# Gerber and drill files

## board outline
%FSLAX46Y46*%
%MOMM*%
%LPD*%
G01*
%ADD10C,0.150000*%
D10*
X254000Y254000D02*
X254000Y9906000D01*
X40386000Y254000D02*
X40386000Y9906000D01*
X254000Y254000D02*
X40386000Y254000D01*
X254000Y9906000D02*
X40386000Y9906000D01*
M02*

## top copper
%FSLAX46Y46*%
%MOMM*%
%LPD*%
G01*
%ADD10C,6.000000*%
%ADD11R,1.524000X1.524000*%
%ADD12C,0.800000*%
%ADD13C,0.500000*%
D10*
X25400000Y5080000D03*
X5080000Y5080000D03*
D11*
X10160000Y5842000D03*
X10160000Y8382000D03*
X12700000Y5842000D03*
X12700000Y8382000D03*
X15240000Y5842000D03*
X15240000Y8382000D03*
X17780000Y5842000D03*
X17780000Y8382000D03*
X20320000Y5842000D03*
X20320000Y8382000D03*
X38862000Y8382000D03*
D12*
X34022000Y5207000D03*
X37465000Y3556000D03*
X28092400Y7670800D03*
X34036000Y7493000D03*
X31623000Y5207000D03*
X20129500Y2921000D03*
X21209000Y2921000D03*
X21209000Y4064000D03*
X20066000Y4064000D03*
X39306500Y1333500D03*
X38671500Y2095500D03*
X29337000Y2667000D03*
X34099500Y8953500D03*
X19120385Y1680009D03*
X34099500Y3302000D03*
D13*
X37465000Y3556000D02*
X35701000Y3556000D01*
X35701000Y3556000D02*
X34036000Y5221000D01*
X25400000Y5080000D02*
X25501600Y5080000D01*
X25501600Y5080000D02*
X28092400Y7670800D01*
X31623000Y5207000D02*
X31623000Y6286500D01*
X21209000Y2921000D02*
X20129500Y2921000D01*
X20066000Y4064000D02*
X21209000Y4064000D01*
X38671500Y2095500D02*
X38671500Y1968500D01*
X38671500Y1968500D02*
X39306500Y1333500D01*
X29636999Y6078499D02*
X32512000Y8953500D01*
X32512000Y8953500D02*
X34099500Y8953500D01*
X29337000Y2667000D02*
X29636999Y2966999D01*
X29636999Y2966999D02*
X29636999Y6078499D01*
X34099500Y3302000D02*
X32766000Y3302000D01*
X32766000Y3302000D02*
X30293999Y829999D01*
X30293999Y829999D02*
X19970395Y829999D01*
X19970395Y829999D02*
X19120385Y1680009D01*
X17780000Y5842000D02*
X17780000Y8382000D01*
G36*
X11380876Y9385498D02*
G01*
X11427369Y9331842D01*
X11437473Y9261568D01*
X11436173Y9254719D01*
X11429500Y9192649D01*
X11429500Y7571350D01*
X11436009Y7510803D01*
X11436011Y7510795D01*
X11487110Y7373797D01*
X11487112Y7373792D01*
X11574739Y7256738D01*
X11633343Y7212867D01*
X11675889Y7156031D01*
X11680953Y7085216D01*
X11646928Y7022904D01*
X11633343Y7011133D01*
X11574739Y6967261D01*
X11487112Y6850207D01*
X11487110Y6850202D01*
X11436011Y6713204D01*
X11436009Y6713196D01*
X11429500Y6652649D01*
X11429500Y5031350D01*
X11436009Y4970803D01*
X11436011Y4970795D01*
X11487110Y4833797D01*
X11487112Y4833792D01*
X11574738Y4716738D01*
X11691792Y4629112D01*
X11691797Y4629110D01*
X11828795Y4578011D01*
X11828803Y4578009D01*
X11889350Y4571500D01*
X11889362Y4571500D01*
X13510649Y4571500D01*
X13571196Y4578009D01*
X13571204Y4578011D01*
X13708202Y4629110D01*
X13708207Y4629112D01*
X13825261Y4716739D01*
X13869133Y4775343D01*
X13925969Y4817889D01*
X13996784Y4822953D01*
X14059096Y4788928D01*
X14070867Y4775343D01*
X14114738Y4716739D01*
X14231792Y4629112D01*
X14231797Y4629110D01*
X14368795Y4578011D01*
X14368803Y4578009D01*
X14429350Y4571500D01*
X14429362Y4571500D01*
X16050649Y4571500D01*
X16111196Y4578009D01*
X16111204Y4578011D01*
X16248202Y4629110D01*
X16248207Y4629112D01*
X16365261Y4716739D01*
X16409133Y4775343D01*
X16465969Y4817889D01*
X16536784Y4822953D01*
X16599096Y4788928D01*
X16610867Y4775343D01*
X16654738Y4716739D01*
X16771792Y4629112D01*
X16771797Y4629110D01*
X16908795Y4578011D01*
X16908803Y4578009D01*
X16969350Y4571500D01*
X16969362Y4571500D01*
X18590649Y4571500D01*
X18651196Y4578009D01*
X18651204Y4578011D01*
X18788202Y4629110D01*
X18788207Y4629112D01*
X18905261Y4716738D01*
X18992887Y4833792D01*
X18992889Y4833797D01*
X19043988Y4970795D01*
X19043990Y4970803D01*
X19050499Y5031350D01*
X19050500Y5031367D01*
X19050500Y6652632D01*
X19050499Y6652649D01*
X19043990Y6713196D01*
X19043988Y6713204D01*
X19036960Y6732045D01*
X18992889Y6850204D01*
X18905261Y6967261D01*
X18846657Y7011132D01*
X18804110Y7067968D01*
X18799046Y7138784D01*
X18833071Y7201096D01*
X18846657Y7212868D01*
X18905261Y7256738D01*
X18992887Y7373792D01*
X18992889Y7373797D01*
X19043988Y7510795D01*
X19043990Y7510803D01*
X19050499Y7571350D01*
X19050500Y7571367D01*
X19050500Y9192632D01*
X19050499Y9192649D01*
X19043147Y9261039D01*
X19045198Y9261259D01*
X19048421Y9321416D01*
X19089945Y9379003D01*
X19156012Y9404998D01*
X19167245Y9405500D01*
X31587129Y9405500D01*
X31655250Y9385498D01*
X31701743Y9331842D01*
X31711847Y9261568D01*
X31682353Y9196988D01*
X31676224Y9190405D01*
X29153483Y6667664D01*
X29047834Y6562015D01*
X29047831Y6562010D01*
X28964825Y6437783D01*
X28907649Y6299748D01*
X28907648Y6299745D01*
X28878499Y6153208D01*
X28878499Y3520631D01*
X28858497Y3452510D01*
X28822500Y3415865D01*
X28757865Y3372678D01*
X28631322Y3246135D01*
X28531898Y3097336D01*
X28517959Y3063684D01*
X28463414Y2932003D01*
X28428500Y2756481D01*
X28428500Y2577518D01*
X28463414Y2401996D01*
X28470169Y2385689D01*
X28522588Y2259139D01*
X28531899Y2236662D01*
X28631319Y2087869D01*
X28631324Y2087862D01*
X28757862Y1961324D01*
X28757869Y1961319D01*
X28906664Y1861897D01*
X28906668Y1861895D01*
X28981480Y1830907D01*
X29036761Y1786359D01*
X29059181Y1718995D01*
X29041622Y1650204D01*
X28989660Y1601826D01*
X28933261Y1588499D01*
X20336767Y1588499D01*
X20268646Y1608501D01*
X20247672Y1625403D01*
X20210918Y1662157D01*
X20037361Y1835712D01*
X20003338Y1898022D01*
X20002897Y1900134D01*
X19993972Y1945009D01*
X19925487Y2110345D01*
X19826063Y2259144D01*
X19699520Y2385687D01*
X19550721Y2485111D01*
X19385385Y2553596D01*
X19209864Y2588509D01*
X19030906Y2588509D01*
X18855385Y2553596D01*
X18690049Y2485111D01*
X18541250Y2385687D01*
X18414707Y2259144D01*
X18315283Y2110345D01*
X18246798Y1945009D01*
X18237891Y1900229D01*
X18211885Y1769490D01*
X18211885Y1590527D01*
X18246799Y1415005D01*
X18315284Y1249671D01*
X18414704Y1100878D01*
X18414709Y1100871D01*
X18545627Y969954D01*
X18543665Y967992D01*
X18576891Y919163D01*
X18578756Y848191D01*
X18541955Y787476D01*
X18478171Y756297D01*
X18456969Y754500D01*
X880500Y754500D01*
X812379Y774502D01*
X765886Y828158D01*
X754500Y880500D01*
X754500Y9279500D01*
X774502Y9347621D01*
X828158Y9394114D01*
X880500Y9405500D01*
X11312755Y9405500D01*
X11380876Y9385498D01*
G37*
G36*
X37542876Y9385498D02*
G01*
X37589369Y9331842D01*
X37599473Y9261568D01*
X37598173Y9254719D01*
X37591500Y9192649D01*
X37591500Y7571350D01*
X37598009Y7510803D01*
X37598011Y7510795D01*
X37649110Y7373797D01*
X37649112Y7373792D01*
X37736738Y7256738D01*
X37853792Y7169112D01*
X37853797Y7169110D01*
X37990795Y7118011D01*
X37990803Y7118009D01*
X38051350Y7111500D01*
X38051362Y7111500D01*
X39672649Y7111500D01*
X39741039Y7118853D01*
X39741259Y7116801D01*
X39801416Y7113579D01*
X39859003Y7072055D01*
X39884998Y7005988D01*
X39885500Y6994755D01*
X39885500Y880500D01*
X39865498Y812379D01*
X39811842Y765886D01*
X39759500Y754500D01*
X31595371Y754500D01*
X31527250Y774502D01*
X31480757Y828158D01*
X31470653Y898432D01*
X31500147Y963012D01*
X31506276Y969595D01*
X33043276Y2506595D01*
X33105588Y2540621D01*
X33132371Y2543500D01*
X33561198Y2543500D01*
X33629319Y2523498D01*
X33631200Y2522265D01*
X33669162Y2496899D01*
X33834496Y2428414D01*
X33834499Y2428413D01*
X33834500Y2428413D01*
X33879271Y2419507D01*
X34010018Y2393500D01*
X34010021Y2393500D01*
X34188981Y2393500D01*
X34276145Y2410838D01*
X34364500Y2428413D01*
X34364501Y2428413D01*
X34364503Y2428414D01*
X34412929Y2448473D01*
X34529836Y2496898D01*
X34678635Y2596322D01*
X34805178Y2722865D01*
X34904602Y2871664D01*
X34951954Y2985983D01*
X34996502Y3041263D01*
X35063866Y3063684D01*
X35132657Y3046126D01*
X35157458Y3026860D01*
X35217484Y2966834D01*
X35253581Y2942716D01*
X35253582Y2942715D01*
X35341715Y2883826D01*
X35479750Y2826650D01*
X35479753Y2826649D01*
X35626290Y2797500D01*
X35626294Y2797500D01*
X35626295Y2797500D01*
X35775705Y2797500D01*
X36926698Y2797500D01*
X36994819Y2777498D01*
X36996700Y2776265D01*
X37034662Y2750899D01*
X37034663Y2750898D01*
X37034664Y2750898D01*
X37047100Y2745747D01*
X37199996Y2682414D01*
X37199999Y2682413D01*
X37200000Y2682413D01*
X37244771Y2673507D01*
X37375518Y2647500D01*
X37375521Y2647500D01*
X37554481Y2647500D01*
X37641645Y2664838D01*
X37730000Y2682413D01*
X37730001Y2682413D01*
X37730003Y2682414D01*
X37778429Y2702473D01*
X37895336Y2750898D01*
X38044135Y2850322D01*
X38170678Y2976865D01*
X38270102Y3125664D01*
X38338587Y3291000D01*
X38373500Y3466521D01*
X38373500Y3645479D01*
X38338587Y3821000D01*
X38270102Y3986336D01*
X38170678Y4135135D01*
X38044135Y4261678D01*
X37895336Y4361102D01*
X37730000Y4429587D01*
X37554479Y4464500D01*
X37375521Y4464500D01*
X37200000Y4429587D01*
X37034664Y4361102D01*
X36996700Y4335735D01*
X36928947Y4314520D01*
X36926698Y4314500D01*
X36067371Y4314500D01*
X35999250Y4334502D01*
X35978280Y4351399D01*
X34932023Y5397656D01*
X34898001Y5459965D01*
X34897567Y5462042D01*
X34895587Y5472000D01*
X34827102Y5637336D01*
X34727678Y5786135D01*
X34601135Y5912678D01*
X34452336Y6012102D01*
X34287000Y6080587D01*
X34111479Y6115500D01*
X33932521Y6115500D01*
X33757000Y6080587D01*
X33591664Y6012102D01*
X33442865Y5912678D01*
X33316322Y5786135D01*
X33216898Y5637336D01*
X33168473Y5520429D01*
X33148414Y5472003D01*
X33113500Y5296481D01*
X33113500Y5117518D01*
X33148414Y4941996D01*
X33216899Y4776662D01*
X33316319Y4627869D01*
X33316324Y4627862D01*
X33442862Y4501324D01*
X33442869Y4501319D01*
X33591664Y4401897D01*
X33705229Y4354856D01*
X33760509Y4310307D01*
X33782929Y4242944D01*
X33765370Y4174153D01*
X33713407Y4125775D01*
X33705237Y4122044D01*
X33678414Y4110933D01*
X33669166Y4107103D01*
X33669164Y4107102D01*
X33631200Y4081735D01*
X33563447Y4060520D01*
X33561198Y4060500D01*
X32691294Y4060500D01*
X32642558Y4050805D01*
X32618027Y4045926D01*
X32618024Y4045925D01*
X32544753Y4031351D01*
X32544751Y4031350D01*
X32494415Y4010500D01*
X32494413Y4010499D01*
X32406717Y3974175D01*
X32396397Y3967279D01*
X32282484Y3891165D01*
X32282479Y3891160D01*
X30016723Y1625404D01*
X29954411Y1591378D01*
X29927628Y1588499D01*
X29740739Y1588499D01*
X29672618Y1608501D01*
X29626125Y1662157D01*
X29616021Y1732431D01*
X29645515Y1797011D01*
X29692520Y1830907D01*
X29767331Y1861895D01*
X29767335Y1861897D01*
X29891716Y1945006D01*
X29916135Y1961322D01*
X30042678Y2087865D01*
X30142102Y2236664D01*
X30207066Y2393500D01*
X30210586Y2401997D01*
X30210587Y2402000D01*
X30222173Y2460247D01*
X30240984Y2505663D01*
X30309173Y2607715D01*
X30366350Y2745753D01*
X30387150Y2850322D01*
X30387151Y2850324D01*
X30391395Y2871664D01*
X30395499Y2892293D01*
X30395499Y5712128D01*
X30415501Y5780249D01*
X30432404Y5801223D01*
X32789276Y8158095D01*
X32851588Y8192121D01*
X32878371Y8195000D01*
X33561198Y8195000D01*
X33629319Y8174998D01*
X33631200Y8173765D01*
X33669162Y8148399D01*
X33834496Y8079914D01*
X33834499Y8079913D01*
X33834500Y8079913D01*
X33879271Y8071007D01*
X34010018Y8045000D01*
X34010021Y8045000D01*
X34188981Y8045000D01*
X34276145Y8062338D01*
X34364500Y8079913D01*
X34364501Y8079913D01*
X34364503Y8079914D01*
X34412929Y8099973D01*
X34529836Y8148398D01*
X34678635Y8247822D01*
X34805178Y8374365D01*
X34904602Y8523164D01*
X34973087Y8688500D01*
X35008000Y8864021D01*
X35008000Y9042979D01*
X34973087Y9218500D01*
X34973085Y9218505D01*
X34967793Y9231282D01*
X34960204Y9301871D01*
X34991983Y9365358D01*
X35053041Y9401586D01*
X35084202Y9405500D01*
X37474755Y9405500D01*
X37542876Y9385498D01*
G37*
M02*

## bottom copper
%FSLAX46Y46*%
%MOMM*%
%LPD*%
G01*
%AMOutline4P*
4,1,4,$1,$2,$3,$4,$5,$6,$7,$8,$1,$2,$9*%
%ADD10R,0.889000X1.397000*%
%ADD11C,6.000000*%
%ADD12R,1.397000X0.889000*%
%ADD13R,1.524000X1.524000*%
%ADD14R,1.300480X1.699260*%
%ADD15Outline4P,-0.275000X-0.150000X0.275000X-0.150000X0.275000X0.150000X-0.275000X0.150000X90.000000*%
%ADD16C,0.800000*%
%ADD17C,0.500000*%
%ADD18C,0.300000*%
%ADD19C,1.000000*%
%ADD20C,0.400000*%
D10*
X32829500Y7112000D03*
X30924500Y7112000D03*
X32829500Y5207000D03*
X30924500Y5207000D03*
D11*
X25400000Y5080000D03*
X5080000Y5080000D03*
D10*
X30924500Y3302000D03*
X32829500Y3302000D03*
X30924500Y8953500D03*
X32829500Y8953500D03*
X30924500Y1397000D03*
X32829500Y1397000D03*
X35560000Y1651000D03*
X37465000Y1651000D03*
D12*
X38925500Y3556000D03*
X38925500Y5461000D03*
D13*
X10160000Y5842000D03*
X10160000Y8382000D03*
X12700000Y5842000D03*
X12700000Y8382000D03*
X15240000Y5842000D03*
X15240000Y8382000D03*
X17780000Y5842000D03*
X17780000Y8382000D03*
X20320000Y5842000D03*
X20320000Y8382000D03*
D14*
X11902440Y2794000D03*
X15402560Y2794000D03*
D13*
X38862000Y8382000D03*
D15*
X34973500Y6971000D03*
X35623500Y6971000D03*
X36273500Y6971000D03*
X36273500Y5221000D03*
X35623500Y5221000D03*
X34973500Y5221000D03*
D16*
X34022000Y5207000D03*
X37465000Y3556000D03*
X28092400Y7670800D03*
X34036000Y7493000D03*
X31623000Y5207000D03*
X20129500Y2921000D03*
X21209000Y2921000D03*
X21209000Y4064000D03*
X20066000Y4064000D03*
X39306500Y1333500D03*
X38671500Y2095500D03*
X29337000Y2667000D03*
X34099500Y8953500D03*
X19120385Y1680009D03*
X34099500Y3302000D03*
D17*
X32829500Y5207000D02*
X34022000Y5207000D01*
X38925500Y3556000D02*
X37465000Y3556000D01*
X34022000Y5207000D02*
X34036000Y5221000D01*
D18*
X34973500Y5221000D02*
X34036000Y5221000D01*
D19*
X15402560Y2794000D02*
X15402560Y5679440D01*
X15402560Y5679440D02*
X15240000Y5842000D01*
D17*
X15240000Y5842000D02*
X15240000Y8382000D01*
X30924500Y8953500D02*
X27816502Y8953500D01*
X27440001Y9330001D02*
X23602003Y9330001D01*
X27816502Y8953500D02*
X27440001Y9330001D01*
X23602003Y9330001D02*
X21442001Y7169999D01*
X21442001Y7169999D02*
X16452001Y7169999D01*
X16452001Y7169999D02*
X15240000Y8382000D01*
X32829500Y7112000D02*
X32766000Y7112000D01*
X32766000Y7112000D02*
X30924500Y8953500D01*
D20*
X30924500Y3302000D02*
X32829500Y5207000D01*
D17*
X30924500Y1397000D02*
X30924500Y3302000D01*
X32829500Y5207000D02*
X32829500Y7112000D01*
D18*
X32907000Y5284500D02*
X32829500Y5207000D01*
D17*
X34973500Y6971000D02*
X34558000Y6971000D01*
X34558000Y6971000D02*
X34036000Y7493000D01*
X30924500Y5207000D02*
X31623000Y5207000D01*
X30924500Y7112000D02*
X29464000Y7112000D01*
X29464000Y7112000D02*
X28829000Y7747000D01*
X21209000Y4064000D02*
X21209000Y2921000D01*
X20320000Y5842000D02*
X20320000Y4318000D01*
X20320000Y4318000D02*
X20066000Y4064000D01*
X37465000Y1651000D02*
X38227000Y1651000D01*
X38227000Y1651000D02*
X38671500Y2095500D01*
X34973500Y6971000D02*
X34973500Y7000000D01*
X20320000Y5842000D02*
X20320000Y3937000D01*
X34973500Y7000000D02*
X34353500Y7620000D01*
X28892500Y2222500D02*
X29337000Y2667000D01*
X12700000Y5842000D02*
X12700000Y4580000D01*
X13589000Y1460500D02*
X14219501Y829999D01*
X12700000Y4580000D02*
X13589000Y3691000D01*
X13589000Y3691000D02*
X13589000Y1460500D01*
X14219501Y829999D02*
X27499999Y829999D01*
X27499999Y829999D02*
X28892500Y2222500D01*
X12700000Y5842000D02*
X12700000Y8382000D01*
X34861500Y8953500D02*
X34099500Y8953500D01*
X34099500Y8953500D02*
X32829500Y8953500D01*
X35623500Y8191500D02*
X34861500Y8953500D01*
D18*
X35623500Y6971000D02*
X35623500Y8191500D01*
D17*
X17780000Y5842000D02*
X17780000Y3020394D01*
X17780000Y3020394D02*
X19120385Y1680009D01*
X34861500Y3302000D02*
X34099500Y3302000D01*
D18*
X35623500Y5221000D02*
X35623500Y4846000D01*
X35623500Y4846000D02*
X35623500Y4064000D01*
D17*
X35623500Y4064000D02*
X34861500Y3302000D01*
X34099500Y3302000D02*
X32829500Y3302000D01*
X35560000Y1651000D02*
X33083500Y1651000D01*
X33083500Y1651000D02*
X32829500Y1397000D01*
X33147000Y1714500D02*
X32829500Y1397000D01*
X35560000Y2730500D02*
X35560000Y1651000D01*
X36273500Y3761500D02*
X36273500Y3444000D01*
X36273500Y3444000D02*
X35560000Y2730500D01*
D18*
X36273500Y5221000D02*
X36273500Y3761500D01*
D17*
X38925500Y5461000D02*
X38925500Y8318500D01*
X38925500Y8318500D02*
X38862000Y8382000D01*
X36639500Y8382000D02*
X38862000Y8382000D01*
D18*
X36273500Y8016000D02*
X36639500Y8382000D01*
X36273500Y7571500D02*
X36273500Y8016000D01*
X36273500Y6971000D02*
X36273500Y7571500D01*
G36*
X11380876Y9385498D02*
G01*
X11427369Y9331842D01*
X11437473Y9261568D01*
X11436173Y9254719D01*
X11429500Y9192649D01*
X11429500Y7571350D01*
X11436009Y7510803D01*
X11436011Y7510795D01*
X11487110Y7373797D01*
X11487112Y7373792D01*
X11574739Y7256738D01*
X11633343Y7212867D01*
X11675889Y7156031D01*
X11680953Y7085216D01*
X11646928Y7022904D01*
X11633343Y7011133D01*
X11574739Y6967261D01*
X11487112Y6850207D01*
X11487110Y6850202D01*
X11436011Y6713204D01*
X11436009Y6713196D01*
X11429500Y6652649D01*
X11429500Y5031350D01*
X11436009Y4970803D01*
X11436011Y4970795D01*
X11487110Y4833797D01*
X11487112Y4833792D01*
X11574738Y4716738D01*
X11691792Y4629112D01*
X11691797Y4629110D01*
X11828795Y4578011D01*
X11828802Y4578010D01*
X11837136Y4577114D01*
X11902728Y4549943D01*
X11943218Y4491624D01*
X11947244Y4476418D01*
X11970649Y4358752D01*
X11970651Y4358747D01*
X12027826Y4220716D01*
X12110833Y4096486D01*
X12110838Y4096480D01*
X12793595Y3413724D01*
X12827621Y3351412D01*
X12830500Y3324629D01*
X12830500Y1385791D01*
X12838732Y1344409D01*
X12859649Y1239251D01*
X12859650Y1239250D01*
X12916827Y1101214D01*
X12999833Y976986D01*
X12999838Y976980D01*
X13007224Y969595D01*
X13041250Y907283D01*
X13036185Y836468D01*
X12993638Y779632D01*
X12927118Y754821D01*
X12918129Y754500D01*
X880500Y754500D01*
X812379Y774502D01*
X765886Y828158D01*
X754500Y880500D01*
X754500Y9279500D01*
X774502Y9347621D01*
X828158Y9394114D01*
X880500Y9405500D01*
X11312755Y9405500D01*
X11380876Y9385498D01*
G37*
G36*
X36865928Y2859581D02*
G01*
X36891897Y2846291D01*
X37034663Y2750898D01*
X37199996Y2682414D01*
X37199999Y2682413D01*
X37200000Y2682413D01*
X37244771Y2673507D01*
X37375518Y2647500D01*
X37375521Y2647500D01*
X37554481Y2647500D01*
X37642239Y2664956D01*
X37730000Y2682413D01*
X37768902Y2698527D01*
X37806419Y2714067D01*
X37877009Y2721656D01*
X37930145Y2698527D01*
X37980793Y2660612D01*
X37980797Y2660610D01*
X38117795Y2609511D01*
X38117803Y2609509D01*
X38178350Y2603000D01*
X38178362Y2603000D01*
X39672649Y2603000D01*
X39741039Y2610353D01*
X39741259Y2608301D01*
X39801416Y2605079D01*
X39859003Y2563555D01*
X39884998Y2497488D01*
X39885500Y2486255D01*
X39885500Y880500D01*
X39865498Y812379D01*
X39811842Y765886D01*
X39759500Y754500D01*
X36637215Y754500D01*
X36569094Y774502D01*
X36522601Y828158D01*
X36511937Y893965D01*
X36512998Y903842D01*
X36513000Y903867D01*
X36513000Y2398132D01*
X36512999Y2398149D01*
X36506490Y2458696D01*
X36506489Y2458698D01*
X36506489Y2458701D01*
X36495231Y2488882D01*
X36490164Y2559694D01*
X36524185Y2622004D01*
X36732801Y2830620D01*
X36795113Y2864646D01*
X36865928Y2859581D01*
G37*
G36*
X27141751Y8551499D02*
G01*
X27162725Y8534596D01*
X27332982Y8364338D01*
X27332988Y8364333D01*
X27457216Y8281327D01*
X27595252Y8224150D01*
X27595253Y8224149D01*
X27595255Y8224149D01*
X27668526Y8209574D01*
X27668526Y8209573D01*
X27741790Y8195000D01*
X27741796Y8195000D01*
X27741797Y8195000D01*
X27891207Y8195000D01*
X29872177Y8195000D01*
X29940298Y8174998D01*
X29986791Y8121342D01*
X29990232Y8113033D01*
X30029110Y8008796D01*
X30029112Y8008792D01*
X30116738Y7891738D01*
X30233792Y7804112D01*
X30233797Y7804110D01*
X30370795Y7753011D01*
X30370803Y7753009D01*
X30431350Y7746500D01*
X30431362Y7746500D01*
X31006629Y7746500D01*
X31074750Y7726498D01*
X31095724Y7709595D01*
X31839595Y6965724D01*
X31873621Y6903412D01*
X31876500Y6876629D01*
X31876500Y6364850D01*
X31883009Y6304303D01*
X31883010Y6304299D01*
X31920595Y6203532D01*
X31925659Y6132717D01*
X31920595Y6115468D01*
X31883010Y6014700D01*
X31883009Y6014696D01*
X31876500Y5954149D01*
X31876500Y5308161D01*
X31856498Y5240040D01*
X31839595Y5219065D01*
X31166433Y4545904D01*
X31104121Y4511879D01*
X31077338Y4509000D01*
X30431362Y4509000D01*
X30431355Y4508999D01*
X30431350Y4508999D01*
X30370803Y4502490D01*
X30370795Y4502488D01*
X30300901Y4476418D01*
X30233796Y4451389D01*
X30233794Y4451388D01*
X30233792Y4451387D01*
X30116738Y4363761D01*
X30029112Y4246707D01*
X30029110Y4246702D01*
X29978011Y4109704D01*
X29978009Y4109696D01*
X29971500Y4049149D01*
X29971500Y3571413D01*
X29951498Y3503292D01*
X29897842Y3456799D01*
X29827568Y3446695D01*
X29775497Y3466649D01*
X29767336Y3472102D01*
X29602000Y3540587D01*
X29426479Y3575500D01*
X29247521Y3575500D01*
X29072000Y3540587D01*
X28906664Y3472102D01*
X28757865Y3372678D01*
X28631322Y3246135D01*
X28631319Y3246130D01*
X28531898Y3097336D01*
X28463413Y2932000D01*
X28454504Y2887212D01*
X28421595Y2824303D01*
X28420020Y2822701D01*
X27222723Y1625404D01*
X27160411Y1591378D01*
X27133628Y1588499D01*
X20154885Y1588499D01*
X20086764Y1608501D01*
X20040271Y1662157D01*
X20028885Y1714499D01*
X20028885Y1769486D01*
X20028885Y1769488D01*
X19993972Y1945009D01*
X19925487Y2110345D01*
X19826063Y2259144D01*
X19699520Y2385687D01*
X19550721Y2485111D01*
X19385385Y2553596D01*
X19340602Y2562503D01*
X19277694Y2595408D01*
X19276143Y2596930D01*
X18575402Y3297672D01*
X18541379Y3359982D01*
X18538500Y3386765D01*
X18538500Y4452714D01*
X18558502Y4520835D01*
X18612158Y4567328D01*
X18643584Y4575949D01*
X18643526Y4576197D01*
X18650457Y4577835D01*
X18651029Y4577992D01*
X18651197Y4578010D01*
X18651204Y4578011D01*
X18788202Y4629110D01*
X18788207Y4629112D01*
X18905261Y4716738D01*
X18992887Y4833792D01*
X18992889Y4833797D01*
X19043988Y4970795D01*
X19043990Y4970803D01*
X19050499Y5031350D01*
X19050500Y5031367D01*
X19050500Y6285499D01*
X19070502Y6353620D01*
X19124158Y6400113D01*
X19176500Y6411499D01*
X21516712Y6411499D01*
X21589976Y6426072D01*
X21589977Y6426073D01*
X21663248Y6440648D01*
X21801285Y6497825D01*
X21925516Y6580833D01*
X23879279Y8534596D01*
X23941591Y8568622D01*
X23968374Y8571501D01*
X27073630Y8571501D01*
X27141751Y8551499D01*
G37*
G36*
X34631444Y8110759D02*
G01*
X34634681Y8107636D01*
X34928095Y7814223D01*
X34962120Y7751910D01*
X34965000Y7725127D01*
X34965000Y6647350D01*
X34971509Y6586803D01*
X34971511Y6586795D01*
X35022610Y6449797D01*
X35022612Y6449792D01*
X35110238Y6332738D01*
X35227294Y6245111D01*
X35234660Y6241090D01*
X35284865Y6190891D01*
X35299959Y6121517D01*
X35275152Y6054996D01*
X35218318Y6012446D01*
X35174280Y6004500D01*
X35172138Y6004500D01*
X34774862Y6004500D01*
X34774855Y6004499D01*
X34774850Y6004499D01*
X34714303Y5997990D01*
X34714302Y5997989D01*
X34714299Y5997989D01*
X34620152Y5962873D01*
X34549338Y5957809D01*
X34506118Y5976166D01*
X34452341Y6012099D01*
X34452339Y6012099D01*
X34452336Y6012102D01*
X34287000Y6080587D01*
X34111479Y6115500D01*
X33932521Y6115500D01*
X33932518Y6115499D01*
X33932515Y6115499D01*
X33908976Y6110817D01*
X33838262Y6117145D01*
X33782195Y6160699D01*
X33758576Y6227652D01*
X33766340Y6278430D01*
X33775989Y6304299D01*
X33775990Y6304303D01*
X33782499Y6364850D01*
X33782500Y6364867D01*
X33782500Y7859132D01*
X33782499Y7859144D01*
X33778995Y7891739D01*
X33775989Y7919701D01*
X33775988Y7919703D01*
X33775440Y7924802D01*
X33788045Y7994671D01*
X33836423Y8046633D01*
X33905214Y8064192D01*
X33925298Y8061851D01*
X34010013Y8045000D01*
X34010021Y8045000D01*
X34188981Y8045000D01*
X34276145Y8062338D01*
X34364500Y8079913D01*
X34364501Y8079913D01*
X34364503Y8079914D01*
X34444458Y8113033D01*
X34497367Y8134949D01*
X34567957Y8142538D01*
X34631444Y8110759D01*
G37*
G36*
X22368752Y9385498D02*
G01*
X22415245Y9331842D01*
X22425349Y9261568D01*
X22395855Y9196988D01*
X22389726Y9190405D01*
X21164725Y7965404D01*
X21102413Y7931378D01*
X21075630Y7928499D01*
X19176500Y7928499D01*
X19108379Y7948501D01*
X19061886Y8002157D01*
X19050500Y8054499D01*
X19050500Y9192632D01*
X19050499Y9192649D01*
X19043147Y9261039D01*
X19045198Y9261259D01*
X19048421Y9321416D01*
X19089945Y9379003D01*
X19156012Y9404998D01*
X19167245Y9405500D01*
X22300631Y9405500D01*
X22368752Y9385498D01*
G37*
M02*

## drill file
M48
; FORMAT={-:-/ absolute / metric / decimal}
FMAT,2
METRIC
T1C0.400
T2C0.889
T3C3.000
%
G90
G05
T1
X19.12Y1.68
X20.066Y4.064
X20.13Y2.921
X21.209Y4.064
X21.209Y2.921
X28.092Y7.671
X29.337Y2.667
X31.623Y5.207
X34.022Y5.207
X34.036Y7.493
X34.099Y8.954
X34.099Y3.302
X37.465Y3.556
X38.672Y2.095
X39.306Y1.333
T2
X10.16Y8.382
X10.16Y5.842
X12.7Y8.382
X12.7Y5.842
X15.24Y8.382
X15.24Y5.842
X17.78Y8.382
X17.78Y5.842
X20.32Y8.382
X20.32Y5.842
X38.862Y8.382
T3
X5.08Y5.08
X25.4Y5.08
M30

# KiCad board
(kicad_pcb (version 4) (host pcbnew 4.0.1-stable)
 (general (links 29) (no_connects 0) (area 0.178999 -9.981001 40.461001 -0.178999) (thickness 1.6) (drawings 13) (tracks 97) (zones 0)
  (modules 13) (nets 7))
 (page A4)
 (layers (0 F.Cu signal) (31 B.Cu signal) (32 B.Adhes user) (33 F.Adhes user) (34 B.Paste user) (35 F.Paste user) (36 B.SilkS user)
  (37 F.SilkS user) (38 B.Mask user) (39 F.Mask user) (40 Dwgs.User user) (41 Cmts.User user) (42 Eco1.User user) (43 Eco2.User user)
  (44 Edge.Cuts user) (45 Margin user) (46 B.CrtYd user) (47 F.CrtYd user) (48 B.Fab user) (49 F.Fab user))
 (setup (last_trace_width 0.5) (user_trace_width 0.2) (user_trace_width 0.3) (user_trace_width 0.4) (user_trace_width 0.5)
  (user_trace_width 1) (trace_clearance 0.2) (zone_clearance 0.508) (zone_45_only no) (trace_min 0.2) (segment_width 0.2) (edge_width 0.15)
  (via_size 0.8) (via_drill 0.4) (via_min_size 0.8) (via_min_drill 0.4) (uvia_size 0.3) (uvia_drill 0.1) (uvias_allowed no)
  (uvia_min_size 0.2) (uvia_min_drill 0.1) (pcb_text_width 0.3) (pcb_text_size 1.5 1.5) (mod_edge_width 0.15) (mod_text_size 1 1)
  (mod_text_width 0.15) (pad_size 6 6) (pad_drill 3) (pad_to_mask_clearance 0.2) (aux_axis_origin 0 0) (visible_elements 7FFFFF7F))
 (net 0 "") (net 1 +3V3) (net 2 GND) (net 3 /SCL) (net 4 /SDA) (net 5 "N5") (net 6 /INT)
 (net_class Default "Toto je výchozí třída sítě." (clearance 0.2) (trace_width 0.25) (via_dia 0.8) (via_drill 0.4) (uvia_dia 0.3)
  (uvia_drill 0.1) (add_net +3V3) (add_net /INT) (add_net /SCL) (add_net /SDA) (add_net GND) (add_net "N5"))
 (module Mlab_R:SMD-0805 (layer B.Cu) (at 31.877 -7.112 180)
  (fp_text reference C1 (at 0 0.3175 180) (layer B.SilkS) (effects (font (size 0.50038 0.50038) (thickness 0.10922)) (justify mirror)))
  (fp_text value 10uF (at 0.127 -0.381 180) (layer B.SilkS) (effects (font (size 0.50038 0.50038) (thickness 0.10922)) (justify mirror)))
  (pad 1 smd rect (at -0.9525 0 180) (size 0.889 1.397) (layers B.Cu B.Paste B.Mask) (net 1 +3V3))
  (pad 2 smd rect (at 0.9525 0 180) (size 0.889 1.397) (layers B.Cu B.Paste B.Mask) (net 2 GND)))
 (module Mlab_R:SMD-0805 (layer B.Cu) (at 31.877 -5.207 180)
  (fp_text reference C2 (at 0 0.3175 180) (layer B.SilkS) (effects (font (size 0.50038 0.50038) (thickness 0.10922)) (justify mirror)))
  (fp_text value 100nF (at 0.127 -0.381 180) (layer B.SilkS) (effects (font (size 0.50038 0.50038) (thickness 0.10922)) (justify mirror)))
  (pad 1 smd rect (at -0.9525 0 180) (size 0.889 1.397) (layers B.Cu B.Paste B.Mask) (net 1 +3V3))
  (pad 2 smd rect (at 0.9525 0 180) (size 0.889 1.397) (layers B.Cu B.Paste B.Mask) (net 2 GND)))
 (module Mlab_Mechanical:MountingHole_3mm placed (layer F.Cu) (at 25.4 -5.08)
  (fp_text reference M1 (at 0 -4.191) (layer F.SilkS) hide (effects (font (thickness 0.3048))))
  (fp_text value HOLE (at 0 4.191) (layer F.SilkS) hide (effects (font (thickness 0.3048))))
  (pad 1 thru_hole circle (at 0 0) (size 6 6) (drill 3) (layers *.Cu *.Adhes *.Mask) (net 2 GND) (clearance 1) (zone_connect 2)))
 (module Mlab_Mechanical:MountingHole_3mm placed (layer F.Cu) (at 5.08 -5.08)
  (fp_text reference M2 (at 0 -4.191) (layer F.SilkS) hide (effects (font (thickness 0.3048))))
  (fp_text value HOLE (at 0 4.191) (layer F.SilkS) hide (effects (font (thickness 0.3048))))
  (pad 1 thru_hole circle (at 0 0) (size 6 6) (drill 3) (layers *.Cu *.Adhes *.Mask) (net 2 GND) (clearance 1) (zone_connect 2)))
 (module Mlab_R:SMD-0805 (layer B.Cu) (at 31.877 -3.302)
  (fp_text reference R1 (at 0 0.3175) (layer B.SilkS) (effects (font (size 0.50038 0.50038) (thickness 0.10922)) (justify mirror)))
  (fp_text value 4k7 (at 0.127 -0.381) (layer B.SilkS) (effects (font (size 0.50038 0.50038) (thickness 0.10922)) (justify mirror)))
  (pad 1 smd rect (at -0.9525 0) (size 0.889 1.397) (layers B.Cu B.Paste B.Mask) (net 1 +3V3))
  (pad 2 smd rect (at 0.9525 0) (size 0.889 1.397) (layers B.Cu B.Paste B.Mask) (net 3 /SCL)))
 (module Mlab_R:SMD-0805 (layer B.Cu) (at 31.877 -8.9535)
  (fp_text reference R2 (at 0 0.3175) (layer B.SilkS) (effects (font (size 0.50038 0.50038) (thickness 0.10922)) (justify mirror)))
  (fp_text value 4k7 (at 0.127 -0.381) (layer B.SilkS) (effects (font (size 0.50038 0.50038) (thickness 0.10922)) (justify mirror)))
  (pad 1 smd rect (at -0.9525 0) (size 0.889 1.397) (layers B.Cu B.Paste B.Mask) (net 1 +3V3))
  (pad 2 smd rect (at 0.9525 0) (size 0.889 1.397) (layers B.Cu B.Paste B.Mask) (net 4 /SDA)))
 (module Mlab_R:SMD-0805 (layer B.Cu) (at 31.877 -1.397)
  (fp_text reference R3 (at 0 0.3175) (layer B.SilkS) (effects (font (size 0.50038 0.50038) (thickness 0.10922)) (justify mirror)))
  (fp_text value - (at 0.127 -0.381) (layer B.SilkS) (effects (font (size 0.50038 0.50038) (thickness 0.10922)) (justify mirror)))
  (pad 1 smd rect (at -0.9525 0) (size 0.889 1.397) (layers B.Cu B.Paste B.Mask) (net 1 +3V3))
  (pad 2 smd rect (at 0.9525 0) (size 0.889 1.397) (layers B.Cu B.Paste B.Mask) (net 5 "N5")))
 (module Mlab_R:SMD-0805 (layer B.Cu) (at 36.5125 -1.651)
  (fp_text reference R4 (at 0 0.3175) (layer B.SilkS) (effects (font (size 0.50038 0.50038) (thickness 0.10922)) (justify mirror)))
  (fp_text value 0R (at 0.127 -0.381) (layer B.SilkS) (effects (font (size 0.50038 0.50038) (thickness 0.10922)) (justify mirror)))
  (pad 1 smd rect (at -0.9525 0) (size 0.889 1.397) (layers B.Cu B.Paste B.Mask) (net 5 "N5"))
  (pad 2 smd rect (at 0.9525 0) (size 0.889 1.397) (layers B.Cu B.Paste B.Mask) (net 2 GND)))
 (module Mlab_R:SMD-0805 (layer B.Cu) (at 38.9255 -4.5085 90)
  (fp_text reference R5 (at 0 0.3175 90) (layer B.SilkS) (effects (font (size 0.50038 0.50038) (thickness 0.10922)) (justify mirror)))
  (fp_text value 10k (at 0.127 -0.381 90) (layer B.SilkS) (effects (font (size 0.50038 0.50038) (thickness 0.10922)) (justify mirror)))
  (pad 1 smd rect (at -0.9525 0 90) (size 0.889 1.397) (layers B.Cu B.Paste B.Mask) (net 1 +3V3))
  (pad 2 smd rect (at 0.9525 0 90) (size 0.889 1.397) (layers B.Cu B.Paste B.Mask) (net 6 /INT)))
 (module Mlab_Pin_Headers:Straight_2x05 (layer F.Cu) (at 15.24 -7.112 90)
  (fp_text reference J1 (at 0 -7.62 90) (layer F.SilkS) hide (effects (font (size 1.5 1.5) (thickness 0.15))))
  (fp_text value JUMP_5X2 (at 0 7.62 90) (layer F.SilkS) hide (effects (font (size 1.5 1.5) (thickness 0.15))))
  (pad 1 thru_hole rect (at -1.27 -5.08 90) (size 1.524 1.524) (drill 0.889) (layers *.Cu *.Mask F.SilkS) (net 2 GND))
  (pad 2 thru_hole rect (at 1.27 -5.08 90) (size 1.524 1.524) (drill 0.889) (layers *.Cu *.Mask F.SilkS) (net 2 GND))
  (pad 3 thru_hole rect (at -1.27 -2.54 90) (size 1.524 1.524) (drill 0.889) (layers *.Cu *.Mask F.SilkS) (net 4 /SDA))
  (pad 4 thru_hole rect (at 1.27 -2.54 90) (size 1.524 1.524) (drill 0.889) (layers *.Cu *.Mask F.SilkS) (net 4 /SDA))
  (pad 5 thru_hole rect (at -1.27 0 90) (size 1.524 1.524) (drill 0.889) (layers *.Cu *.Mask F.SilkS) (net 1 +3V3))
  (pad 6 thru_hole rect (at 1.27 0 90) (size 1.524 1.524) (drill 0.889) (layers *.Cu *.Mask F.SilkS) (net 1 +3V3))
  (pad 7 thru_hole rect (at -1.27 2.54 90) (size 1.524 1.524) (drill 0.889) (layers *.Cu *.Mask F.SilkS) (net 3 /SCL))
  (pad 8 thru_hole rect (at 1.27 2.54 90) (size 1.524 1.524) (drill 0.889) (layers *.Cu *.Mask F.SilkS) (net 3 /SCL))
  (pad 9 thru_hole rect (at -1.27 5.08 90) (size 1.524 1.524) (drill 0.889) (layers *.Cu *.Mask F.SilkS) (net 2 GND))
  (pad 10 thru_hole rect (at 1.27 5.08 90) (size 1.524 1.524) (drill 0.889) (layers *.Cu *.Mask F.SilkS) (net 2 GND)))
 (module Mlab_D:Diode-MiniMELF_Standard (layer B.Cu) (at 13.6525 -2.794)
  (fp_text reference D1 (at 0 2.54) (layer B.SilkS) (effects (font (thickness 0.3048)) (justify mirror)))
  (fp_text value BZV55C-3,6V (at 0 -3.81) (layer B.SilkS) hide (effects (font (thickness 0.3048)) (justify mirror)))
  (pad 1 smd rect (at -1.75006 0) (size 1.30048 1.69926) (layers B.Cu B.Paste B.Mask) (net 2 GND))
  (pad 2 smd rect (at 1.75006 0) (size 1.30048 1.69926) (layers B.Cu B.Paste B.Mask) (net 1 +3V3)))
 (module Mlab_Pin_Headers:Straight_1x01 (layer F.Cu) (at 38.862 -8.382)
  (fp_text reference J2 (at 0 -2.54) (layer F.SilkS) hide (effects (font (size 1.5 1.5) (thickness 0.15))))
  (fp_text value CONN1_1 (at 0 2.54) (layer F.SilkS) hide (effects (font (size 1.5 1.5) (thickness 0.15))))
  (pad 1 thru_hole rect (at 0 0) (size 1.524 1.524) (drill 0.889) (layers *.Cu *.Mask F.SilkS) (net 6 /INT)))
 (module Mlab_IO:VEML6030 (layer B.Cu) (at 35.6235 -6.096 90)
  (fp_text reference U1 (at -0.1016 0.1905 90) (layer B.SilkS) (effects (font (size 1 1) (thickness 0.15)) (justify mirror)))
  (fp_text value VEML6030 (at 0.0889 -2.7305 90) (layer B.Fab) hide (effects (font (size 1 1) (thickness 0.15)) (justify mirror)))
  (pad 1 smd trapezoid (at 0.875 -0.65 90) (size 0.55 0.3) (layers B.Cu B.Paste B.Mask) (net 2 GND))
  (pad 2 smd trapezoid (at 0.875 0 90) (size 0.55 0.3) (layers B.Cu B.Paste B.Mask) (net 4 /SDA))
  (pad 3 smd trapezoid (at 0.875 0.65 90) (size 0.55 0.3) (layers B.Cu B.Paste B.Mask) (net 6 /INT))
  (pad 4 smd trapezoid (at -0.875 0.65 90) (size 0.55 0.3) (layers B.Cu B.Paste B.Mask) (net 5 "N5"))
  (pad 5 smd trapezoid (at -0.875 0 90) (size 0.55 0.3) (layers B.Cu B.Paste B.Mask) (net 3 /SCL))
  (pad 6 smd trapezoid (at -0.875 -0.65 90) (size 0.55 0.3) (layers B.Cu B.Paste B.Mask) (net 1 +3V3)))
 (gr_line (start 0.254 -0.254) (end 0.254 -9.906) (angle 90) (layer Edge.Cuts) (width 0.15))
 (gr_line (start 40.386 -0.254) (end 40.386 -9.906) (angle 90) (layer Edge.Cuts) (width 0.15))
 (gr_line (start 0.254 -0.254) (end 40.386 -0.254) (angle 90) (layer Edge.Cuts) (width 0.15))
 (gr_line (start 0.254 -9.906) (end 40.386 -9.906) (angle 90) (layer Edge.Cuts) (width 0.15))
 (segment (start 32.8295 -5.207) (end 34.022 -5.207) (width 0.5) (layer B.Cu) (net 1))
 (via (at 34.022 -5.207) (size 0.8) (drill 0.4) (layers F.Cu B.Cu) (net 1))
 (segment (start 38.9255 -3.556) (end 37.465 -3.556) (width 0.5) (layer B.Cu) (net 1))
 (via (at 37.465 -3.556) (size 0.8) (drill 0.4) (layers F.Cu B.Cu) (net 1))
 (segment (start 34.022 -5.207) (end 34.036 -5.221) (width 0.5) (layer B.Cu) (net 1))
 (segment (start 34.9735 -5.221) (end 34.036 -5.221) (width 0.3) (layer B.Cu) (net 1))
 (segment (start 37.465 -3.556) (end 35.701 -3.556) (width 0.5) (layer F.Cu) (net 1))
 (segment (start 35.701 -3.556) (end 34.036 -5.221) (width 0.5) (layer F.Cu) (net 1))
 (segment (start 15.40256 -2.794) (end 15.40256 -5.67944) (width 1) (layer B.Cu) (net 1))
 (segment (start 15.40256 -5.67944) (end 15.24 -5.842) (width 1) (layer B.Cu) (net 1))
 (segment (start 15.24 -5.842) (end 15.24 -8.382) (width 0.5) (layer B.Cu) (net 1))
 (segment (start 30.9245 -8.9535) (end 27.816502 -8.9535) (width 0.5) (layer B.Cu) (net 1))
 (segment (start 27.440001 -9.330001) (end 23.602003 -9.330001) (width 0.5) (layer B.Cu) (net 1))
 (segment (start 27.816502 -8.9535) (end 27.440001 -9.330001) (width 0.5) (layer B.Cu) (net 1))
 (segment (start 23.602003 -9.330001) (end 21.442001 -7.169999) (width 0.5) (layer B.Cu) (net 1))
 (segment (start 21.442001 -7.169999) (end 16.452001 -7.169999) (width 0.5) (layer B.Cu) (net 1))
 (segment (start 16.452001 -7.169999) (end 15.24 -8.382) (width 0.5) (layer B.Cu) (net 1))
 (segment (start 32.8295 -7.112) (end 32.766 -7.112) (width 0.5) (layer B.Cu) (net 1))
 (segment (start 32.766 -7.112) (end 30.9245 -8.9535) (width 0.5) (layer B.Cu) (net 1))
 (segment (start 30.9245 -3.302) (end 32.8295 -5.207) (width 0.4) (layer B.Cu) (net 1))
 (segment (start 30.9245 -1.397) (end 30.9245 -3.302) (width 0.5) (layer B.Cu) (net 1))
 (segment (start 32.8295 -5.207) (end 32.8295 -7.112) (width 0.5) (layer B.Cu) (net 1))
 (segment (start 32.907 -5.2845) (end 32.8295 -5.207) (width 0.3) (layer B.Cu) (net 1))
 (segment (start 25.4 -5.08) (end 25.5016 -5.08) (width 0.5) (layer F.Cu) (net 2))
 (segment (start 25.5016 -5.08) (end 28.0924 -7.6708) (width 0.5) (layer F.Cu) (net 2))
 (via (at 28.0924 -7.6708) (size 0.8) (drill 0.4) (layers F.Cu B.Cu) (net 2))
 (segment (start 34.9735 -6.971) (end 34.558 -6.971) (width 0.5) (layer B.Cu) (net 2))
 (segment (start 34.558 -6.971) (end 34.036 -7.493) (width 0.5) (layer B.Cu) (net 2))
 (via (at 34.036 -7.493) (size 0.8) (drill 0.4) (layers F.Cu B.Cu) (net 2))
 (segment (start 31.623 -5.207) (end 31.623 -6.2865) (width 0.5) (layer F.Cu) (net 2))
 (segment (start 30.9245 -5.207) (end 31.623 -5.207) (width 0.5) (layer B.Cu) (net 2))
 (via (at 31.623 -5.207) (size 0.8) (drill 0.4) (layers F.Cu B.Cu) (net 2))
 (segment (start 30.9245 -7.112) (end 29.464 -7.112) (width 0.5) (layer B.Cu) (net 2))
 (segment (start 29.464 -7.112) (end 28.829 -7.747) (width 0.5) (layer B.Cu) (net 2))
 (segment (start 21.209 -2.921) (end 20.1295 -2.921) (width 0.5) (layer F.Cu) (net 2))
 (via (at 20.1295 -2.921) (size 0.8) (drill 0.4) (layers F.Cu B.Cu) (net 2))
 (segment (start 21.209 -4.064) (end 21.209 -2.921) (width 0.5) (layer B.Cu) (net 2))
 (via (at 21.209 -2.921) (size 0.8) (drill 0.4) (layers F.Cu B.Cu) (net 2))
 (segment (start 20.066 -4.064) (end 21.209 -4.064) (width 0.5) (layer F.Cu) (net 2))
 (via (at 21.209 -4.064) (size 0.8) (drill 0.4) (layers F.Cu B.Cu) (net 2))
 (segment (start 20.32 -5.842) (end 20.32 -4.318) (width 0.5) (layer B.Cu) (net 2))
 (segment (start 20.32 -4.318) (end 20.066 -4.064) (width 0.5) (layer B.Cu) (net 2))
 (via (at 20.066 -4.064) (size 0.8) (drill 0.4) (layers F.Cu B.Cu) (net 2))
 (segment (start 38.6715 -2.0955) (end 38.6715 -1.9685) (width 0.5) (layer F.Cu) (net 2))
 (segment (start 38.6715 -1.9685) (end 39.3065 -1.3335) (width 0.5) (layer F.Cu) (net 2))
 (via (at 39.3065 -1.3335) (size 0.8) (drill 0.4) (layers F.Cu B.Cu) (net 2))
 (segment (start 37.465 -1.651) (end 38.227 -1.651) (width 0.5) (layer B.Cu) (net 2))
 (segment (start 38.227 -1.651) (end 38.6715 -2.0955) (width 0.5) (layer B.Cu) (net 2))
 (via (at 38.6715 -2.0955) (size 0.8) (drill 0.4) (layers F.Cu B.Cu) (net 2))
 (segment (start 34.9735 -6.971) (end 34.9735 -7) (width 0.5) (layer B.Cu) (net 2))
 (segment (start 20.32 -5.842) (end 20.32 -3.937) (width 0.5) (layer B.Cu) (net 2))
 (segment (start 34.9735 -7) (end 34.3535 -7.62) (width 0.5) (layer B.Cu) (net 2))
 (segment (start 28.8925 -2.2225) (end 29.337 -2.667) (width 0.5) (layer B.Cu) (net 4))
 (via (at 29.337 -2.667) (size 0.8) (drill 0.4) (layers F.Cu B.Cu) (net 4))
 (segment (start 12.7 -5.842) (end 12.7 -4.58) (width 0.5) (layer B.Cu) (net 4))
 (segment (start 13.589 -1.4605) (end 14.219501 -0.829999) (width 0.5) (layer B.Cu) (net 4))
 (segment (start 12.7 -4.58) (end 13.589 -3.691) (width 0.5) (layer B.Cu) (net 4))
 (segment (start 13.589 -3.691) (end 13.589 -1.4605) (width 0.5) (layer B.Cu) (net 4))
 (segment (start 14.219501 -0.829999) (end 27.499999 -0.829999) (width 0.5) (layer B.Cu) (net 4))
 (segment (start 27.499999 -0.829999) (end 28.8925 -2.2225) (width 0.5) (layer B.Cu) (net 4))
 (via (at 34.0995 -8.9535) (size 0.8) (drill 0.4) (layers F.Cu B.Cu) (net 4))
 (segment (start 12.7 -5.842) (end 12.7 -8.382) (width 0.5) (layer B.Cu) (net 4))
 (segment (start 34.8615 -8.9535) (end 34.0995 -8.9535) (width 0.5) (layer B.Cu) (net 4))
 (segment (start 34.0995 -8.9535) (end 32.8295 -8.9535) (width 0.5) (layer B.Cu) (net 4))
 (segment (start 29.636999 -6.078499) (end 32.512 -8.9535) (width 0.5) (layer F.Cu) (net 4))
 (segment (start 32.512 -8.9535) (end 34.0995 -8.9535) (width 0.5) (layer F.Cu) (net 4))
 (segment (start 29.337 -2.667) (end 29.636999 -2.966999) (width 0.5) (layer F.Cu) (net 4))
 (segment (start 29.636999 -2.966999) (end 29.636999 -6.078499) (width 0.5) (layer F.Cu) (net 4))
 (segment (start 35.6235 -8.1915) (end 34.8615 -8.9535) (width 0.5) (layer B.Cu) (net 4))
 (segment (start 35.6235 -6.971) (end 35.6235 -8.1915) (width 0.3) (layer B.Cu) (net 4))
 (segment (start 34.0995 -3.302) (end 32.766 -3.302) (width 0.5) (layer F.Cu) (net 3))
 (segment (start 32.766 -3.302) (end 30.293999 -0.829999) (width 0.5) (layer F.Cu) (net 3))
 (segment (start 30.293999 -0.829999) (end 19.970395 -0.829999) (width 0.5) (layer F.Cu) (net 3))
 (segment (start 19.970395 -0.829999) (end 19.120385 -1.680009) (width 0.5) (layer F.Cu) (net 3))
 (segment (start 17.78 -5.842) (end 17.78 -3.020394) (width 0.5) (layer B.Cu) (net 3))
 (segment (start 17.78 -3.020394) (end 19.120385 -1.680009) (width 0.5) (layer B.Cu) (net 3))
 (via (at 19.120385 -1.680009) (size 0.8) (drill 0.4) (layers F.Cu B.Cu) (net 3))
 (via (at 34.0995 -3.302) (size 0.8) (drill 0.4) (layers F.Cu B.Cu) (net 3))
 (segment (start 34.8615 -3.302) (end 34.0995 -3.302) (width 0.5) (layer B.Cu) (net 3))
 (segment (start 35.6235 -5.221) (end 35.6235 -4.846) (width 0.3) (layer B.Cu) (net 3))
 (segment (start 35.6235 -4.846) (end 35.6235 -4.064) (width 0.3) (layer B.Cu) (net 3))
 (segment (start 35.6235 -4.064) (end 34.8615 -3.302) (width 0.5) (layer B.Cu) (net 3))
 (segment (start 17.78 -5.842) (end 17.78 -8.382) (width 0.5) (layer F.Cu) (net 3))
 (segment (start 34.0995 -3.302) (end 32.8295 -3.302) (width 0.5) (layer B.Cu) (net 3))
 (segment (start 35.56 -1.651) (end 33.0835 -1.651) (width 0.5) (layer B.Cu) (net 5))
 (segment (start 33.0835 -1.651) (end 32.8295 -1.397) (width 0.5) (layer B.Cu) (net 5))
 (segment (start 33.147 -1.7145) (end 32.8295 -1.397) (width 0.5) (layer B.Cu) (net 5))
 (segment (start 35.56 -2.7305) (end 35.56 -1.651) (width 0.5) (layer B.Cu) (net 5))
 (segment (start 36.2735 -3.7615) (end 36.2735 -3.444) (width 0.5) (layer B.Cu) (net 5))
 (segment (start 36.2735 -3.444) (end 35.56 -2.7305) (width 0.5) (layer B.Cu) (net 5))
 (segment (start 36.2735 -5.221) (end 36.2735 -3.7615) (width 0.3) (layer B.Cu) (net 5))
 (segment (start 38.9255 -5.461) (end 38.9255 -8.3185) (width 0.5) (layer B.Cu) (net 6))
 (segment (start 38.9255 -8.3185) (end 38.862 -8.382) (width 0.5) (layer B.Cu) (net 6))
 (segment (start 36.6395 -8.382) (end 38.862 -8.382) (width 0.5) (layer B.Cu) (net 6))
 (segment (start 36.2735 -8.016) (end 36.6395 -8.382) (width 0.3) (layer B.Cu) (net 6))
 (segment (start 36.2735 -7.5715) (end 36.2735 -8.016) (width 0.3) (layer B.Cu) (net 6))
 (segment (start 36.2735 -6.971) (end 36.2735 -7.5715) (width 0.3) (layer B.Cu) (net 6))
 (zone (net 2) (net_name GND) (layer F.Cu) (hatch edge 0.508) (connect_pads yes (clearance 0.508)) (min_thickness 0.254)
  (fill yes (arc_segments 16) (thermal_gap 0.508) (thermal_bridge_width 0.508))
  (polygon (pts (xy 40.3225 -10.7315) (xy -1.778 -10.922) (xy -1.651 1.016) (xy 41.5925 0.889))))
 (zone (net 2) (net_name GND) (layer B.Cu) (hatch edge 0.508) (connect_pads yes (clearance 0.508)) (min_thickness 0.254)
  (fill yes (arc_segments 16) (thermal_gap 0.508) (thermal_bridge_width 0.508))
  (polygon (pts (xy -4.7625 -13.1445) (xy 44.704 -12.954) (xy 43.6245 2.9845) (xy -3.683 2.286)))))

